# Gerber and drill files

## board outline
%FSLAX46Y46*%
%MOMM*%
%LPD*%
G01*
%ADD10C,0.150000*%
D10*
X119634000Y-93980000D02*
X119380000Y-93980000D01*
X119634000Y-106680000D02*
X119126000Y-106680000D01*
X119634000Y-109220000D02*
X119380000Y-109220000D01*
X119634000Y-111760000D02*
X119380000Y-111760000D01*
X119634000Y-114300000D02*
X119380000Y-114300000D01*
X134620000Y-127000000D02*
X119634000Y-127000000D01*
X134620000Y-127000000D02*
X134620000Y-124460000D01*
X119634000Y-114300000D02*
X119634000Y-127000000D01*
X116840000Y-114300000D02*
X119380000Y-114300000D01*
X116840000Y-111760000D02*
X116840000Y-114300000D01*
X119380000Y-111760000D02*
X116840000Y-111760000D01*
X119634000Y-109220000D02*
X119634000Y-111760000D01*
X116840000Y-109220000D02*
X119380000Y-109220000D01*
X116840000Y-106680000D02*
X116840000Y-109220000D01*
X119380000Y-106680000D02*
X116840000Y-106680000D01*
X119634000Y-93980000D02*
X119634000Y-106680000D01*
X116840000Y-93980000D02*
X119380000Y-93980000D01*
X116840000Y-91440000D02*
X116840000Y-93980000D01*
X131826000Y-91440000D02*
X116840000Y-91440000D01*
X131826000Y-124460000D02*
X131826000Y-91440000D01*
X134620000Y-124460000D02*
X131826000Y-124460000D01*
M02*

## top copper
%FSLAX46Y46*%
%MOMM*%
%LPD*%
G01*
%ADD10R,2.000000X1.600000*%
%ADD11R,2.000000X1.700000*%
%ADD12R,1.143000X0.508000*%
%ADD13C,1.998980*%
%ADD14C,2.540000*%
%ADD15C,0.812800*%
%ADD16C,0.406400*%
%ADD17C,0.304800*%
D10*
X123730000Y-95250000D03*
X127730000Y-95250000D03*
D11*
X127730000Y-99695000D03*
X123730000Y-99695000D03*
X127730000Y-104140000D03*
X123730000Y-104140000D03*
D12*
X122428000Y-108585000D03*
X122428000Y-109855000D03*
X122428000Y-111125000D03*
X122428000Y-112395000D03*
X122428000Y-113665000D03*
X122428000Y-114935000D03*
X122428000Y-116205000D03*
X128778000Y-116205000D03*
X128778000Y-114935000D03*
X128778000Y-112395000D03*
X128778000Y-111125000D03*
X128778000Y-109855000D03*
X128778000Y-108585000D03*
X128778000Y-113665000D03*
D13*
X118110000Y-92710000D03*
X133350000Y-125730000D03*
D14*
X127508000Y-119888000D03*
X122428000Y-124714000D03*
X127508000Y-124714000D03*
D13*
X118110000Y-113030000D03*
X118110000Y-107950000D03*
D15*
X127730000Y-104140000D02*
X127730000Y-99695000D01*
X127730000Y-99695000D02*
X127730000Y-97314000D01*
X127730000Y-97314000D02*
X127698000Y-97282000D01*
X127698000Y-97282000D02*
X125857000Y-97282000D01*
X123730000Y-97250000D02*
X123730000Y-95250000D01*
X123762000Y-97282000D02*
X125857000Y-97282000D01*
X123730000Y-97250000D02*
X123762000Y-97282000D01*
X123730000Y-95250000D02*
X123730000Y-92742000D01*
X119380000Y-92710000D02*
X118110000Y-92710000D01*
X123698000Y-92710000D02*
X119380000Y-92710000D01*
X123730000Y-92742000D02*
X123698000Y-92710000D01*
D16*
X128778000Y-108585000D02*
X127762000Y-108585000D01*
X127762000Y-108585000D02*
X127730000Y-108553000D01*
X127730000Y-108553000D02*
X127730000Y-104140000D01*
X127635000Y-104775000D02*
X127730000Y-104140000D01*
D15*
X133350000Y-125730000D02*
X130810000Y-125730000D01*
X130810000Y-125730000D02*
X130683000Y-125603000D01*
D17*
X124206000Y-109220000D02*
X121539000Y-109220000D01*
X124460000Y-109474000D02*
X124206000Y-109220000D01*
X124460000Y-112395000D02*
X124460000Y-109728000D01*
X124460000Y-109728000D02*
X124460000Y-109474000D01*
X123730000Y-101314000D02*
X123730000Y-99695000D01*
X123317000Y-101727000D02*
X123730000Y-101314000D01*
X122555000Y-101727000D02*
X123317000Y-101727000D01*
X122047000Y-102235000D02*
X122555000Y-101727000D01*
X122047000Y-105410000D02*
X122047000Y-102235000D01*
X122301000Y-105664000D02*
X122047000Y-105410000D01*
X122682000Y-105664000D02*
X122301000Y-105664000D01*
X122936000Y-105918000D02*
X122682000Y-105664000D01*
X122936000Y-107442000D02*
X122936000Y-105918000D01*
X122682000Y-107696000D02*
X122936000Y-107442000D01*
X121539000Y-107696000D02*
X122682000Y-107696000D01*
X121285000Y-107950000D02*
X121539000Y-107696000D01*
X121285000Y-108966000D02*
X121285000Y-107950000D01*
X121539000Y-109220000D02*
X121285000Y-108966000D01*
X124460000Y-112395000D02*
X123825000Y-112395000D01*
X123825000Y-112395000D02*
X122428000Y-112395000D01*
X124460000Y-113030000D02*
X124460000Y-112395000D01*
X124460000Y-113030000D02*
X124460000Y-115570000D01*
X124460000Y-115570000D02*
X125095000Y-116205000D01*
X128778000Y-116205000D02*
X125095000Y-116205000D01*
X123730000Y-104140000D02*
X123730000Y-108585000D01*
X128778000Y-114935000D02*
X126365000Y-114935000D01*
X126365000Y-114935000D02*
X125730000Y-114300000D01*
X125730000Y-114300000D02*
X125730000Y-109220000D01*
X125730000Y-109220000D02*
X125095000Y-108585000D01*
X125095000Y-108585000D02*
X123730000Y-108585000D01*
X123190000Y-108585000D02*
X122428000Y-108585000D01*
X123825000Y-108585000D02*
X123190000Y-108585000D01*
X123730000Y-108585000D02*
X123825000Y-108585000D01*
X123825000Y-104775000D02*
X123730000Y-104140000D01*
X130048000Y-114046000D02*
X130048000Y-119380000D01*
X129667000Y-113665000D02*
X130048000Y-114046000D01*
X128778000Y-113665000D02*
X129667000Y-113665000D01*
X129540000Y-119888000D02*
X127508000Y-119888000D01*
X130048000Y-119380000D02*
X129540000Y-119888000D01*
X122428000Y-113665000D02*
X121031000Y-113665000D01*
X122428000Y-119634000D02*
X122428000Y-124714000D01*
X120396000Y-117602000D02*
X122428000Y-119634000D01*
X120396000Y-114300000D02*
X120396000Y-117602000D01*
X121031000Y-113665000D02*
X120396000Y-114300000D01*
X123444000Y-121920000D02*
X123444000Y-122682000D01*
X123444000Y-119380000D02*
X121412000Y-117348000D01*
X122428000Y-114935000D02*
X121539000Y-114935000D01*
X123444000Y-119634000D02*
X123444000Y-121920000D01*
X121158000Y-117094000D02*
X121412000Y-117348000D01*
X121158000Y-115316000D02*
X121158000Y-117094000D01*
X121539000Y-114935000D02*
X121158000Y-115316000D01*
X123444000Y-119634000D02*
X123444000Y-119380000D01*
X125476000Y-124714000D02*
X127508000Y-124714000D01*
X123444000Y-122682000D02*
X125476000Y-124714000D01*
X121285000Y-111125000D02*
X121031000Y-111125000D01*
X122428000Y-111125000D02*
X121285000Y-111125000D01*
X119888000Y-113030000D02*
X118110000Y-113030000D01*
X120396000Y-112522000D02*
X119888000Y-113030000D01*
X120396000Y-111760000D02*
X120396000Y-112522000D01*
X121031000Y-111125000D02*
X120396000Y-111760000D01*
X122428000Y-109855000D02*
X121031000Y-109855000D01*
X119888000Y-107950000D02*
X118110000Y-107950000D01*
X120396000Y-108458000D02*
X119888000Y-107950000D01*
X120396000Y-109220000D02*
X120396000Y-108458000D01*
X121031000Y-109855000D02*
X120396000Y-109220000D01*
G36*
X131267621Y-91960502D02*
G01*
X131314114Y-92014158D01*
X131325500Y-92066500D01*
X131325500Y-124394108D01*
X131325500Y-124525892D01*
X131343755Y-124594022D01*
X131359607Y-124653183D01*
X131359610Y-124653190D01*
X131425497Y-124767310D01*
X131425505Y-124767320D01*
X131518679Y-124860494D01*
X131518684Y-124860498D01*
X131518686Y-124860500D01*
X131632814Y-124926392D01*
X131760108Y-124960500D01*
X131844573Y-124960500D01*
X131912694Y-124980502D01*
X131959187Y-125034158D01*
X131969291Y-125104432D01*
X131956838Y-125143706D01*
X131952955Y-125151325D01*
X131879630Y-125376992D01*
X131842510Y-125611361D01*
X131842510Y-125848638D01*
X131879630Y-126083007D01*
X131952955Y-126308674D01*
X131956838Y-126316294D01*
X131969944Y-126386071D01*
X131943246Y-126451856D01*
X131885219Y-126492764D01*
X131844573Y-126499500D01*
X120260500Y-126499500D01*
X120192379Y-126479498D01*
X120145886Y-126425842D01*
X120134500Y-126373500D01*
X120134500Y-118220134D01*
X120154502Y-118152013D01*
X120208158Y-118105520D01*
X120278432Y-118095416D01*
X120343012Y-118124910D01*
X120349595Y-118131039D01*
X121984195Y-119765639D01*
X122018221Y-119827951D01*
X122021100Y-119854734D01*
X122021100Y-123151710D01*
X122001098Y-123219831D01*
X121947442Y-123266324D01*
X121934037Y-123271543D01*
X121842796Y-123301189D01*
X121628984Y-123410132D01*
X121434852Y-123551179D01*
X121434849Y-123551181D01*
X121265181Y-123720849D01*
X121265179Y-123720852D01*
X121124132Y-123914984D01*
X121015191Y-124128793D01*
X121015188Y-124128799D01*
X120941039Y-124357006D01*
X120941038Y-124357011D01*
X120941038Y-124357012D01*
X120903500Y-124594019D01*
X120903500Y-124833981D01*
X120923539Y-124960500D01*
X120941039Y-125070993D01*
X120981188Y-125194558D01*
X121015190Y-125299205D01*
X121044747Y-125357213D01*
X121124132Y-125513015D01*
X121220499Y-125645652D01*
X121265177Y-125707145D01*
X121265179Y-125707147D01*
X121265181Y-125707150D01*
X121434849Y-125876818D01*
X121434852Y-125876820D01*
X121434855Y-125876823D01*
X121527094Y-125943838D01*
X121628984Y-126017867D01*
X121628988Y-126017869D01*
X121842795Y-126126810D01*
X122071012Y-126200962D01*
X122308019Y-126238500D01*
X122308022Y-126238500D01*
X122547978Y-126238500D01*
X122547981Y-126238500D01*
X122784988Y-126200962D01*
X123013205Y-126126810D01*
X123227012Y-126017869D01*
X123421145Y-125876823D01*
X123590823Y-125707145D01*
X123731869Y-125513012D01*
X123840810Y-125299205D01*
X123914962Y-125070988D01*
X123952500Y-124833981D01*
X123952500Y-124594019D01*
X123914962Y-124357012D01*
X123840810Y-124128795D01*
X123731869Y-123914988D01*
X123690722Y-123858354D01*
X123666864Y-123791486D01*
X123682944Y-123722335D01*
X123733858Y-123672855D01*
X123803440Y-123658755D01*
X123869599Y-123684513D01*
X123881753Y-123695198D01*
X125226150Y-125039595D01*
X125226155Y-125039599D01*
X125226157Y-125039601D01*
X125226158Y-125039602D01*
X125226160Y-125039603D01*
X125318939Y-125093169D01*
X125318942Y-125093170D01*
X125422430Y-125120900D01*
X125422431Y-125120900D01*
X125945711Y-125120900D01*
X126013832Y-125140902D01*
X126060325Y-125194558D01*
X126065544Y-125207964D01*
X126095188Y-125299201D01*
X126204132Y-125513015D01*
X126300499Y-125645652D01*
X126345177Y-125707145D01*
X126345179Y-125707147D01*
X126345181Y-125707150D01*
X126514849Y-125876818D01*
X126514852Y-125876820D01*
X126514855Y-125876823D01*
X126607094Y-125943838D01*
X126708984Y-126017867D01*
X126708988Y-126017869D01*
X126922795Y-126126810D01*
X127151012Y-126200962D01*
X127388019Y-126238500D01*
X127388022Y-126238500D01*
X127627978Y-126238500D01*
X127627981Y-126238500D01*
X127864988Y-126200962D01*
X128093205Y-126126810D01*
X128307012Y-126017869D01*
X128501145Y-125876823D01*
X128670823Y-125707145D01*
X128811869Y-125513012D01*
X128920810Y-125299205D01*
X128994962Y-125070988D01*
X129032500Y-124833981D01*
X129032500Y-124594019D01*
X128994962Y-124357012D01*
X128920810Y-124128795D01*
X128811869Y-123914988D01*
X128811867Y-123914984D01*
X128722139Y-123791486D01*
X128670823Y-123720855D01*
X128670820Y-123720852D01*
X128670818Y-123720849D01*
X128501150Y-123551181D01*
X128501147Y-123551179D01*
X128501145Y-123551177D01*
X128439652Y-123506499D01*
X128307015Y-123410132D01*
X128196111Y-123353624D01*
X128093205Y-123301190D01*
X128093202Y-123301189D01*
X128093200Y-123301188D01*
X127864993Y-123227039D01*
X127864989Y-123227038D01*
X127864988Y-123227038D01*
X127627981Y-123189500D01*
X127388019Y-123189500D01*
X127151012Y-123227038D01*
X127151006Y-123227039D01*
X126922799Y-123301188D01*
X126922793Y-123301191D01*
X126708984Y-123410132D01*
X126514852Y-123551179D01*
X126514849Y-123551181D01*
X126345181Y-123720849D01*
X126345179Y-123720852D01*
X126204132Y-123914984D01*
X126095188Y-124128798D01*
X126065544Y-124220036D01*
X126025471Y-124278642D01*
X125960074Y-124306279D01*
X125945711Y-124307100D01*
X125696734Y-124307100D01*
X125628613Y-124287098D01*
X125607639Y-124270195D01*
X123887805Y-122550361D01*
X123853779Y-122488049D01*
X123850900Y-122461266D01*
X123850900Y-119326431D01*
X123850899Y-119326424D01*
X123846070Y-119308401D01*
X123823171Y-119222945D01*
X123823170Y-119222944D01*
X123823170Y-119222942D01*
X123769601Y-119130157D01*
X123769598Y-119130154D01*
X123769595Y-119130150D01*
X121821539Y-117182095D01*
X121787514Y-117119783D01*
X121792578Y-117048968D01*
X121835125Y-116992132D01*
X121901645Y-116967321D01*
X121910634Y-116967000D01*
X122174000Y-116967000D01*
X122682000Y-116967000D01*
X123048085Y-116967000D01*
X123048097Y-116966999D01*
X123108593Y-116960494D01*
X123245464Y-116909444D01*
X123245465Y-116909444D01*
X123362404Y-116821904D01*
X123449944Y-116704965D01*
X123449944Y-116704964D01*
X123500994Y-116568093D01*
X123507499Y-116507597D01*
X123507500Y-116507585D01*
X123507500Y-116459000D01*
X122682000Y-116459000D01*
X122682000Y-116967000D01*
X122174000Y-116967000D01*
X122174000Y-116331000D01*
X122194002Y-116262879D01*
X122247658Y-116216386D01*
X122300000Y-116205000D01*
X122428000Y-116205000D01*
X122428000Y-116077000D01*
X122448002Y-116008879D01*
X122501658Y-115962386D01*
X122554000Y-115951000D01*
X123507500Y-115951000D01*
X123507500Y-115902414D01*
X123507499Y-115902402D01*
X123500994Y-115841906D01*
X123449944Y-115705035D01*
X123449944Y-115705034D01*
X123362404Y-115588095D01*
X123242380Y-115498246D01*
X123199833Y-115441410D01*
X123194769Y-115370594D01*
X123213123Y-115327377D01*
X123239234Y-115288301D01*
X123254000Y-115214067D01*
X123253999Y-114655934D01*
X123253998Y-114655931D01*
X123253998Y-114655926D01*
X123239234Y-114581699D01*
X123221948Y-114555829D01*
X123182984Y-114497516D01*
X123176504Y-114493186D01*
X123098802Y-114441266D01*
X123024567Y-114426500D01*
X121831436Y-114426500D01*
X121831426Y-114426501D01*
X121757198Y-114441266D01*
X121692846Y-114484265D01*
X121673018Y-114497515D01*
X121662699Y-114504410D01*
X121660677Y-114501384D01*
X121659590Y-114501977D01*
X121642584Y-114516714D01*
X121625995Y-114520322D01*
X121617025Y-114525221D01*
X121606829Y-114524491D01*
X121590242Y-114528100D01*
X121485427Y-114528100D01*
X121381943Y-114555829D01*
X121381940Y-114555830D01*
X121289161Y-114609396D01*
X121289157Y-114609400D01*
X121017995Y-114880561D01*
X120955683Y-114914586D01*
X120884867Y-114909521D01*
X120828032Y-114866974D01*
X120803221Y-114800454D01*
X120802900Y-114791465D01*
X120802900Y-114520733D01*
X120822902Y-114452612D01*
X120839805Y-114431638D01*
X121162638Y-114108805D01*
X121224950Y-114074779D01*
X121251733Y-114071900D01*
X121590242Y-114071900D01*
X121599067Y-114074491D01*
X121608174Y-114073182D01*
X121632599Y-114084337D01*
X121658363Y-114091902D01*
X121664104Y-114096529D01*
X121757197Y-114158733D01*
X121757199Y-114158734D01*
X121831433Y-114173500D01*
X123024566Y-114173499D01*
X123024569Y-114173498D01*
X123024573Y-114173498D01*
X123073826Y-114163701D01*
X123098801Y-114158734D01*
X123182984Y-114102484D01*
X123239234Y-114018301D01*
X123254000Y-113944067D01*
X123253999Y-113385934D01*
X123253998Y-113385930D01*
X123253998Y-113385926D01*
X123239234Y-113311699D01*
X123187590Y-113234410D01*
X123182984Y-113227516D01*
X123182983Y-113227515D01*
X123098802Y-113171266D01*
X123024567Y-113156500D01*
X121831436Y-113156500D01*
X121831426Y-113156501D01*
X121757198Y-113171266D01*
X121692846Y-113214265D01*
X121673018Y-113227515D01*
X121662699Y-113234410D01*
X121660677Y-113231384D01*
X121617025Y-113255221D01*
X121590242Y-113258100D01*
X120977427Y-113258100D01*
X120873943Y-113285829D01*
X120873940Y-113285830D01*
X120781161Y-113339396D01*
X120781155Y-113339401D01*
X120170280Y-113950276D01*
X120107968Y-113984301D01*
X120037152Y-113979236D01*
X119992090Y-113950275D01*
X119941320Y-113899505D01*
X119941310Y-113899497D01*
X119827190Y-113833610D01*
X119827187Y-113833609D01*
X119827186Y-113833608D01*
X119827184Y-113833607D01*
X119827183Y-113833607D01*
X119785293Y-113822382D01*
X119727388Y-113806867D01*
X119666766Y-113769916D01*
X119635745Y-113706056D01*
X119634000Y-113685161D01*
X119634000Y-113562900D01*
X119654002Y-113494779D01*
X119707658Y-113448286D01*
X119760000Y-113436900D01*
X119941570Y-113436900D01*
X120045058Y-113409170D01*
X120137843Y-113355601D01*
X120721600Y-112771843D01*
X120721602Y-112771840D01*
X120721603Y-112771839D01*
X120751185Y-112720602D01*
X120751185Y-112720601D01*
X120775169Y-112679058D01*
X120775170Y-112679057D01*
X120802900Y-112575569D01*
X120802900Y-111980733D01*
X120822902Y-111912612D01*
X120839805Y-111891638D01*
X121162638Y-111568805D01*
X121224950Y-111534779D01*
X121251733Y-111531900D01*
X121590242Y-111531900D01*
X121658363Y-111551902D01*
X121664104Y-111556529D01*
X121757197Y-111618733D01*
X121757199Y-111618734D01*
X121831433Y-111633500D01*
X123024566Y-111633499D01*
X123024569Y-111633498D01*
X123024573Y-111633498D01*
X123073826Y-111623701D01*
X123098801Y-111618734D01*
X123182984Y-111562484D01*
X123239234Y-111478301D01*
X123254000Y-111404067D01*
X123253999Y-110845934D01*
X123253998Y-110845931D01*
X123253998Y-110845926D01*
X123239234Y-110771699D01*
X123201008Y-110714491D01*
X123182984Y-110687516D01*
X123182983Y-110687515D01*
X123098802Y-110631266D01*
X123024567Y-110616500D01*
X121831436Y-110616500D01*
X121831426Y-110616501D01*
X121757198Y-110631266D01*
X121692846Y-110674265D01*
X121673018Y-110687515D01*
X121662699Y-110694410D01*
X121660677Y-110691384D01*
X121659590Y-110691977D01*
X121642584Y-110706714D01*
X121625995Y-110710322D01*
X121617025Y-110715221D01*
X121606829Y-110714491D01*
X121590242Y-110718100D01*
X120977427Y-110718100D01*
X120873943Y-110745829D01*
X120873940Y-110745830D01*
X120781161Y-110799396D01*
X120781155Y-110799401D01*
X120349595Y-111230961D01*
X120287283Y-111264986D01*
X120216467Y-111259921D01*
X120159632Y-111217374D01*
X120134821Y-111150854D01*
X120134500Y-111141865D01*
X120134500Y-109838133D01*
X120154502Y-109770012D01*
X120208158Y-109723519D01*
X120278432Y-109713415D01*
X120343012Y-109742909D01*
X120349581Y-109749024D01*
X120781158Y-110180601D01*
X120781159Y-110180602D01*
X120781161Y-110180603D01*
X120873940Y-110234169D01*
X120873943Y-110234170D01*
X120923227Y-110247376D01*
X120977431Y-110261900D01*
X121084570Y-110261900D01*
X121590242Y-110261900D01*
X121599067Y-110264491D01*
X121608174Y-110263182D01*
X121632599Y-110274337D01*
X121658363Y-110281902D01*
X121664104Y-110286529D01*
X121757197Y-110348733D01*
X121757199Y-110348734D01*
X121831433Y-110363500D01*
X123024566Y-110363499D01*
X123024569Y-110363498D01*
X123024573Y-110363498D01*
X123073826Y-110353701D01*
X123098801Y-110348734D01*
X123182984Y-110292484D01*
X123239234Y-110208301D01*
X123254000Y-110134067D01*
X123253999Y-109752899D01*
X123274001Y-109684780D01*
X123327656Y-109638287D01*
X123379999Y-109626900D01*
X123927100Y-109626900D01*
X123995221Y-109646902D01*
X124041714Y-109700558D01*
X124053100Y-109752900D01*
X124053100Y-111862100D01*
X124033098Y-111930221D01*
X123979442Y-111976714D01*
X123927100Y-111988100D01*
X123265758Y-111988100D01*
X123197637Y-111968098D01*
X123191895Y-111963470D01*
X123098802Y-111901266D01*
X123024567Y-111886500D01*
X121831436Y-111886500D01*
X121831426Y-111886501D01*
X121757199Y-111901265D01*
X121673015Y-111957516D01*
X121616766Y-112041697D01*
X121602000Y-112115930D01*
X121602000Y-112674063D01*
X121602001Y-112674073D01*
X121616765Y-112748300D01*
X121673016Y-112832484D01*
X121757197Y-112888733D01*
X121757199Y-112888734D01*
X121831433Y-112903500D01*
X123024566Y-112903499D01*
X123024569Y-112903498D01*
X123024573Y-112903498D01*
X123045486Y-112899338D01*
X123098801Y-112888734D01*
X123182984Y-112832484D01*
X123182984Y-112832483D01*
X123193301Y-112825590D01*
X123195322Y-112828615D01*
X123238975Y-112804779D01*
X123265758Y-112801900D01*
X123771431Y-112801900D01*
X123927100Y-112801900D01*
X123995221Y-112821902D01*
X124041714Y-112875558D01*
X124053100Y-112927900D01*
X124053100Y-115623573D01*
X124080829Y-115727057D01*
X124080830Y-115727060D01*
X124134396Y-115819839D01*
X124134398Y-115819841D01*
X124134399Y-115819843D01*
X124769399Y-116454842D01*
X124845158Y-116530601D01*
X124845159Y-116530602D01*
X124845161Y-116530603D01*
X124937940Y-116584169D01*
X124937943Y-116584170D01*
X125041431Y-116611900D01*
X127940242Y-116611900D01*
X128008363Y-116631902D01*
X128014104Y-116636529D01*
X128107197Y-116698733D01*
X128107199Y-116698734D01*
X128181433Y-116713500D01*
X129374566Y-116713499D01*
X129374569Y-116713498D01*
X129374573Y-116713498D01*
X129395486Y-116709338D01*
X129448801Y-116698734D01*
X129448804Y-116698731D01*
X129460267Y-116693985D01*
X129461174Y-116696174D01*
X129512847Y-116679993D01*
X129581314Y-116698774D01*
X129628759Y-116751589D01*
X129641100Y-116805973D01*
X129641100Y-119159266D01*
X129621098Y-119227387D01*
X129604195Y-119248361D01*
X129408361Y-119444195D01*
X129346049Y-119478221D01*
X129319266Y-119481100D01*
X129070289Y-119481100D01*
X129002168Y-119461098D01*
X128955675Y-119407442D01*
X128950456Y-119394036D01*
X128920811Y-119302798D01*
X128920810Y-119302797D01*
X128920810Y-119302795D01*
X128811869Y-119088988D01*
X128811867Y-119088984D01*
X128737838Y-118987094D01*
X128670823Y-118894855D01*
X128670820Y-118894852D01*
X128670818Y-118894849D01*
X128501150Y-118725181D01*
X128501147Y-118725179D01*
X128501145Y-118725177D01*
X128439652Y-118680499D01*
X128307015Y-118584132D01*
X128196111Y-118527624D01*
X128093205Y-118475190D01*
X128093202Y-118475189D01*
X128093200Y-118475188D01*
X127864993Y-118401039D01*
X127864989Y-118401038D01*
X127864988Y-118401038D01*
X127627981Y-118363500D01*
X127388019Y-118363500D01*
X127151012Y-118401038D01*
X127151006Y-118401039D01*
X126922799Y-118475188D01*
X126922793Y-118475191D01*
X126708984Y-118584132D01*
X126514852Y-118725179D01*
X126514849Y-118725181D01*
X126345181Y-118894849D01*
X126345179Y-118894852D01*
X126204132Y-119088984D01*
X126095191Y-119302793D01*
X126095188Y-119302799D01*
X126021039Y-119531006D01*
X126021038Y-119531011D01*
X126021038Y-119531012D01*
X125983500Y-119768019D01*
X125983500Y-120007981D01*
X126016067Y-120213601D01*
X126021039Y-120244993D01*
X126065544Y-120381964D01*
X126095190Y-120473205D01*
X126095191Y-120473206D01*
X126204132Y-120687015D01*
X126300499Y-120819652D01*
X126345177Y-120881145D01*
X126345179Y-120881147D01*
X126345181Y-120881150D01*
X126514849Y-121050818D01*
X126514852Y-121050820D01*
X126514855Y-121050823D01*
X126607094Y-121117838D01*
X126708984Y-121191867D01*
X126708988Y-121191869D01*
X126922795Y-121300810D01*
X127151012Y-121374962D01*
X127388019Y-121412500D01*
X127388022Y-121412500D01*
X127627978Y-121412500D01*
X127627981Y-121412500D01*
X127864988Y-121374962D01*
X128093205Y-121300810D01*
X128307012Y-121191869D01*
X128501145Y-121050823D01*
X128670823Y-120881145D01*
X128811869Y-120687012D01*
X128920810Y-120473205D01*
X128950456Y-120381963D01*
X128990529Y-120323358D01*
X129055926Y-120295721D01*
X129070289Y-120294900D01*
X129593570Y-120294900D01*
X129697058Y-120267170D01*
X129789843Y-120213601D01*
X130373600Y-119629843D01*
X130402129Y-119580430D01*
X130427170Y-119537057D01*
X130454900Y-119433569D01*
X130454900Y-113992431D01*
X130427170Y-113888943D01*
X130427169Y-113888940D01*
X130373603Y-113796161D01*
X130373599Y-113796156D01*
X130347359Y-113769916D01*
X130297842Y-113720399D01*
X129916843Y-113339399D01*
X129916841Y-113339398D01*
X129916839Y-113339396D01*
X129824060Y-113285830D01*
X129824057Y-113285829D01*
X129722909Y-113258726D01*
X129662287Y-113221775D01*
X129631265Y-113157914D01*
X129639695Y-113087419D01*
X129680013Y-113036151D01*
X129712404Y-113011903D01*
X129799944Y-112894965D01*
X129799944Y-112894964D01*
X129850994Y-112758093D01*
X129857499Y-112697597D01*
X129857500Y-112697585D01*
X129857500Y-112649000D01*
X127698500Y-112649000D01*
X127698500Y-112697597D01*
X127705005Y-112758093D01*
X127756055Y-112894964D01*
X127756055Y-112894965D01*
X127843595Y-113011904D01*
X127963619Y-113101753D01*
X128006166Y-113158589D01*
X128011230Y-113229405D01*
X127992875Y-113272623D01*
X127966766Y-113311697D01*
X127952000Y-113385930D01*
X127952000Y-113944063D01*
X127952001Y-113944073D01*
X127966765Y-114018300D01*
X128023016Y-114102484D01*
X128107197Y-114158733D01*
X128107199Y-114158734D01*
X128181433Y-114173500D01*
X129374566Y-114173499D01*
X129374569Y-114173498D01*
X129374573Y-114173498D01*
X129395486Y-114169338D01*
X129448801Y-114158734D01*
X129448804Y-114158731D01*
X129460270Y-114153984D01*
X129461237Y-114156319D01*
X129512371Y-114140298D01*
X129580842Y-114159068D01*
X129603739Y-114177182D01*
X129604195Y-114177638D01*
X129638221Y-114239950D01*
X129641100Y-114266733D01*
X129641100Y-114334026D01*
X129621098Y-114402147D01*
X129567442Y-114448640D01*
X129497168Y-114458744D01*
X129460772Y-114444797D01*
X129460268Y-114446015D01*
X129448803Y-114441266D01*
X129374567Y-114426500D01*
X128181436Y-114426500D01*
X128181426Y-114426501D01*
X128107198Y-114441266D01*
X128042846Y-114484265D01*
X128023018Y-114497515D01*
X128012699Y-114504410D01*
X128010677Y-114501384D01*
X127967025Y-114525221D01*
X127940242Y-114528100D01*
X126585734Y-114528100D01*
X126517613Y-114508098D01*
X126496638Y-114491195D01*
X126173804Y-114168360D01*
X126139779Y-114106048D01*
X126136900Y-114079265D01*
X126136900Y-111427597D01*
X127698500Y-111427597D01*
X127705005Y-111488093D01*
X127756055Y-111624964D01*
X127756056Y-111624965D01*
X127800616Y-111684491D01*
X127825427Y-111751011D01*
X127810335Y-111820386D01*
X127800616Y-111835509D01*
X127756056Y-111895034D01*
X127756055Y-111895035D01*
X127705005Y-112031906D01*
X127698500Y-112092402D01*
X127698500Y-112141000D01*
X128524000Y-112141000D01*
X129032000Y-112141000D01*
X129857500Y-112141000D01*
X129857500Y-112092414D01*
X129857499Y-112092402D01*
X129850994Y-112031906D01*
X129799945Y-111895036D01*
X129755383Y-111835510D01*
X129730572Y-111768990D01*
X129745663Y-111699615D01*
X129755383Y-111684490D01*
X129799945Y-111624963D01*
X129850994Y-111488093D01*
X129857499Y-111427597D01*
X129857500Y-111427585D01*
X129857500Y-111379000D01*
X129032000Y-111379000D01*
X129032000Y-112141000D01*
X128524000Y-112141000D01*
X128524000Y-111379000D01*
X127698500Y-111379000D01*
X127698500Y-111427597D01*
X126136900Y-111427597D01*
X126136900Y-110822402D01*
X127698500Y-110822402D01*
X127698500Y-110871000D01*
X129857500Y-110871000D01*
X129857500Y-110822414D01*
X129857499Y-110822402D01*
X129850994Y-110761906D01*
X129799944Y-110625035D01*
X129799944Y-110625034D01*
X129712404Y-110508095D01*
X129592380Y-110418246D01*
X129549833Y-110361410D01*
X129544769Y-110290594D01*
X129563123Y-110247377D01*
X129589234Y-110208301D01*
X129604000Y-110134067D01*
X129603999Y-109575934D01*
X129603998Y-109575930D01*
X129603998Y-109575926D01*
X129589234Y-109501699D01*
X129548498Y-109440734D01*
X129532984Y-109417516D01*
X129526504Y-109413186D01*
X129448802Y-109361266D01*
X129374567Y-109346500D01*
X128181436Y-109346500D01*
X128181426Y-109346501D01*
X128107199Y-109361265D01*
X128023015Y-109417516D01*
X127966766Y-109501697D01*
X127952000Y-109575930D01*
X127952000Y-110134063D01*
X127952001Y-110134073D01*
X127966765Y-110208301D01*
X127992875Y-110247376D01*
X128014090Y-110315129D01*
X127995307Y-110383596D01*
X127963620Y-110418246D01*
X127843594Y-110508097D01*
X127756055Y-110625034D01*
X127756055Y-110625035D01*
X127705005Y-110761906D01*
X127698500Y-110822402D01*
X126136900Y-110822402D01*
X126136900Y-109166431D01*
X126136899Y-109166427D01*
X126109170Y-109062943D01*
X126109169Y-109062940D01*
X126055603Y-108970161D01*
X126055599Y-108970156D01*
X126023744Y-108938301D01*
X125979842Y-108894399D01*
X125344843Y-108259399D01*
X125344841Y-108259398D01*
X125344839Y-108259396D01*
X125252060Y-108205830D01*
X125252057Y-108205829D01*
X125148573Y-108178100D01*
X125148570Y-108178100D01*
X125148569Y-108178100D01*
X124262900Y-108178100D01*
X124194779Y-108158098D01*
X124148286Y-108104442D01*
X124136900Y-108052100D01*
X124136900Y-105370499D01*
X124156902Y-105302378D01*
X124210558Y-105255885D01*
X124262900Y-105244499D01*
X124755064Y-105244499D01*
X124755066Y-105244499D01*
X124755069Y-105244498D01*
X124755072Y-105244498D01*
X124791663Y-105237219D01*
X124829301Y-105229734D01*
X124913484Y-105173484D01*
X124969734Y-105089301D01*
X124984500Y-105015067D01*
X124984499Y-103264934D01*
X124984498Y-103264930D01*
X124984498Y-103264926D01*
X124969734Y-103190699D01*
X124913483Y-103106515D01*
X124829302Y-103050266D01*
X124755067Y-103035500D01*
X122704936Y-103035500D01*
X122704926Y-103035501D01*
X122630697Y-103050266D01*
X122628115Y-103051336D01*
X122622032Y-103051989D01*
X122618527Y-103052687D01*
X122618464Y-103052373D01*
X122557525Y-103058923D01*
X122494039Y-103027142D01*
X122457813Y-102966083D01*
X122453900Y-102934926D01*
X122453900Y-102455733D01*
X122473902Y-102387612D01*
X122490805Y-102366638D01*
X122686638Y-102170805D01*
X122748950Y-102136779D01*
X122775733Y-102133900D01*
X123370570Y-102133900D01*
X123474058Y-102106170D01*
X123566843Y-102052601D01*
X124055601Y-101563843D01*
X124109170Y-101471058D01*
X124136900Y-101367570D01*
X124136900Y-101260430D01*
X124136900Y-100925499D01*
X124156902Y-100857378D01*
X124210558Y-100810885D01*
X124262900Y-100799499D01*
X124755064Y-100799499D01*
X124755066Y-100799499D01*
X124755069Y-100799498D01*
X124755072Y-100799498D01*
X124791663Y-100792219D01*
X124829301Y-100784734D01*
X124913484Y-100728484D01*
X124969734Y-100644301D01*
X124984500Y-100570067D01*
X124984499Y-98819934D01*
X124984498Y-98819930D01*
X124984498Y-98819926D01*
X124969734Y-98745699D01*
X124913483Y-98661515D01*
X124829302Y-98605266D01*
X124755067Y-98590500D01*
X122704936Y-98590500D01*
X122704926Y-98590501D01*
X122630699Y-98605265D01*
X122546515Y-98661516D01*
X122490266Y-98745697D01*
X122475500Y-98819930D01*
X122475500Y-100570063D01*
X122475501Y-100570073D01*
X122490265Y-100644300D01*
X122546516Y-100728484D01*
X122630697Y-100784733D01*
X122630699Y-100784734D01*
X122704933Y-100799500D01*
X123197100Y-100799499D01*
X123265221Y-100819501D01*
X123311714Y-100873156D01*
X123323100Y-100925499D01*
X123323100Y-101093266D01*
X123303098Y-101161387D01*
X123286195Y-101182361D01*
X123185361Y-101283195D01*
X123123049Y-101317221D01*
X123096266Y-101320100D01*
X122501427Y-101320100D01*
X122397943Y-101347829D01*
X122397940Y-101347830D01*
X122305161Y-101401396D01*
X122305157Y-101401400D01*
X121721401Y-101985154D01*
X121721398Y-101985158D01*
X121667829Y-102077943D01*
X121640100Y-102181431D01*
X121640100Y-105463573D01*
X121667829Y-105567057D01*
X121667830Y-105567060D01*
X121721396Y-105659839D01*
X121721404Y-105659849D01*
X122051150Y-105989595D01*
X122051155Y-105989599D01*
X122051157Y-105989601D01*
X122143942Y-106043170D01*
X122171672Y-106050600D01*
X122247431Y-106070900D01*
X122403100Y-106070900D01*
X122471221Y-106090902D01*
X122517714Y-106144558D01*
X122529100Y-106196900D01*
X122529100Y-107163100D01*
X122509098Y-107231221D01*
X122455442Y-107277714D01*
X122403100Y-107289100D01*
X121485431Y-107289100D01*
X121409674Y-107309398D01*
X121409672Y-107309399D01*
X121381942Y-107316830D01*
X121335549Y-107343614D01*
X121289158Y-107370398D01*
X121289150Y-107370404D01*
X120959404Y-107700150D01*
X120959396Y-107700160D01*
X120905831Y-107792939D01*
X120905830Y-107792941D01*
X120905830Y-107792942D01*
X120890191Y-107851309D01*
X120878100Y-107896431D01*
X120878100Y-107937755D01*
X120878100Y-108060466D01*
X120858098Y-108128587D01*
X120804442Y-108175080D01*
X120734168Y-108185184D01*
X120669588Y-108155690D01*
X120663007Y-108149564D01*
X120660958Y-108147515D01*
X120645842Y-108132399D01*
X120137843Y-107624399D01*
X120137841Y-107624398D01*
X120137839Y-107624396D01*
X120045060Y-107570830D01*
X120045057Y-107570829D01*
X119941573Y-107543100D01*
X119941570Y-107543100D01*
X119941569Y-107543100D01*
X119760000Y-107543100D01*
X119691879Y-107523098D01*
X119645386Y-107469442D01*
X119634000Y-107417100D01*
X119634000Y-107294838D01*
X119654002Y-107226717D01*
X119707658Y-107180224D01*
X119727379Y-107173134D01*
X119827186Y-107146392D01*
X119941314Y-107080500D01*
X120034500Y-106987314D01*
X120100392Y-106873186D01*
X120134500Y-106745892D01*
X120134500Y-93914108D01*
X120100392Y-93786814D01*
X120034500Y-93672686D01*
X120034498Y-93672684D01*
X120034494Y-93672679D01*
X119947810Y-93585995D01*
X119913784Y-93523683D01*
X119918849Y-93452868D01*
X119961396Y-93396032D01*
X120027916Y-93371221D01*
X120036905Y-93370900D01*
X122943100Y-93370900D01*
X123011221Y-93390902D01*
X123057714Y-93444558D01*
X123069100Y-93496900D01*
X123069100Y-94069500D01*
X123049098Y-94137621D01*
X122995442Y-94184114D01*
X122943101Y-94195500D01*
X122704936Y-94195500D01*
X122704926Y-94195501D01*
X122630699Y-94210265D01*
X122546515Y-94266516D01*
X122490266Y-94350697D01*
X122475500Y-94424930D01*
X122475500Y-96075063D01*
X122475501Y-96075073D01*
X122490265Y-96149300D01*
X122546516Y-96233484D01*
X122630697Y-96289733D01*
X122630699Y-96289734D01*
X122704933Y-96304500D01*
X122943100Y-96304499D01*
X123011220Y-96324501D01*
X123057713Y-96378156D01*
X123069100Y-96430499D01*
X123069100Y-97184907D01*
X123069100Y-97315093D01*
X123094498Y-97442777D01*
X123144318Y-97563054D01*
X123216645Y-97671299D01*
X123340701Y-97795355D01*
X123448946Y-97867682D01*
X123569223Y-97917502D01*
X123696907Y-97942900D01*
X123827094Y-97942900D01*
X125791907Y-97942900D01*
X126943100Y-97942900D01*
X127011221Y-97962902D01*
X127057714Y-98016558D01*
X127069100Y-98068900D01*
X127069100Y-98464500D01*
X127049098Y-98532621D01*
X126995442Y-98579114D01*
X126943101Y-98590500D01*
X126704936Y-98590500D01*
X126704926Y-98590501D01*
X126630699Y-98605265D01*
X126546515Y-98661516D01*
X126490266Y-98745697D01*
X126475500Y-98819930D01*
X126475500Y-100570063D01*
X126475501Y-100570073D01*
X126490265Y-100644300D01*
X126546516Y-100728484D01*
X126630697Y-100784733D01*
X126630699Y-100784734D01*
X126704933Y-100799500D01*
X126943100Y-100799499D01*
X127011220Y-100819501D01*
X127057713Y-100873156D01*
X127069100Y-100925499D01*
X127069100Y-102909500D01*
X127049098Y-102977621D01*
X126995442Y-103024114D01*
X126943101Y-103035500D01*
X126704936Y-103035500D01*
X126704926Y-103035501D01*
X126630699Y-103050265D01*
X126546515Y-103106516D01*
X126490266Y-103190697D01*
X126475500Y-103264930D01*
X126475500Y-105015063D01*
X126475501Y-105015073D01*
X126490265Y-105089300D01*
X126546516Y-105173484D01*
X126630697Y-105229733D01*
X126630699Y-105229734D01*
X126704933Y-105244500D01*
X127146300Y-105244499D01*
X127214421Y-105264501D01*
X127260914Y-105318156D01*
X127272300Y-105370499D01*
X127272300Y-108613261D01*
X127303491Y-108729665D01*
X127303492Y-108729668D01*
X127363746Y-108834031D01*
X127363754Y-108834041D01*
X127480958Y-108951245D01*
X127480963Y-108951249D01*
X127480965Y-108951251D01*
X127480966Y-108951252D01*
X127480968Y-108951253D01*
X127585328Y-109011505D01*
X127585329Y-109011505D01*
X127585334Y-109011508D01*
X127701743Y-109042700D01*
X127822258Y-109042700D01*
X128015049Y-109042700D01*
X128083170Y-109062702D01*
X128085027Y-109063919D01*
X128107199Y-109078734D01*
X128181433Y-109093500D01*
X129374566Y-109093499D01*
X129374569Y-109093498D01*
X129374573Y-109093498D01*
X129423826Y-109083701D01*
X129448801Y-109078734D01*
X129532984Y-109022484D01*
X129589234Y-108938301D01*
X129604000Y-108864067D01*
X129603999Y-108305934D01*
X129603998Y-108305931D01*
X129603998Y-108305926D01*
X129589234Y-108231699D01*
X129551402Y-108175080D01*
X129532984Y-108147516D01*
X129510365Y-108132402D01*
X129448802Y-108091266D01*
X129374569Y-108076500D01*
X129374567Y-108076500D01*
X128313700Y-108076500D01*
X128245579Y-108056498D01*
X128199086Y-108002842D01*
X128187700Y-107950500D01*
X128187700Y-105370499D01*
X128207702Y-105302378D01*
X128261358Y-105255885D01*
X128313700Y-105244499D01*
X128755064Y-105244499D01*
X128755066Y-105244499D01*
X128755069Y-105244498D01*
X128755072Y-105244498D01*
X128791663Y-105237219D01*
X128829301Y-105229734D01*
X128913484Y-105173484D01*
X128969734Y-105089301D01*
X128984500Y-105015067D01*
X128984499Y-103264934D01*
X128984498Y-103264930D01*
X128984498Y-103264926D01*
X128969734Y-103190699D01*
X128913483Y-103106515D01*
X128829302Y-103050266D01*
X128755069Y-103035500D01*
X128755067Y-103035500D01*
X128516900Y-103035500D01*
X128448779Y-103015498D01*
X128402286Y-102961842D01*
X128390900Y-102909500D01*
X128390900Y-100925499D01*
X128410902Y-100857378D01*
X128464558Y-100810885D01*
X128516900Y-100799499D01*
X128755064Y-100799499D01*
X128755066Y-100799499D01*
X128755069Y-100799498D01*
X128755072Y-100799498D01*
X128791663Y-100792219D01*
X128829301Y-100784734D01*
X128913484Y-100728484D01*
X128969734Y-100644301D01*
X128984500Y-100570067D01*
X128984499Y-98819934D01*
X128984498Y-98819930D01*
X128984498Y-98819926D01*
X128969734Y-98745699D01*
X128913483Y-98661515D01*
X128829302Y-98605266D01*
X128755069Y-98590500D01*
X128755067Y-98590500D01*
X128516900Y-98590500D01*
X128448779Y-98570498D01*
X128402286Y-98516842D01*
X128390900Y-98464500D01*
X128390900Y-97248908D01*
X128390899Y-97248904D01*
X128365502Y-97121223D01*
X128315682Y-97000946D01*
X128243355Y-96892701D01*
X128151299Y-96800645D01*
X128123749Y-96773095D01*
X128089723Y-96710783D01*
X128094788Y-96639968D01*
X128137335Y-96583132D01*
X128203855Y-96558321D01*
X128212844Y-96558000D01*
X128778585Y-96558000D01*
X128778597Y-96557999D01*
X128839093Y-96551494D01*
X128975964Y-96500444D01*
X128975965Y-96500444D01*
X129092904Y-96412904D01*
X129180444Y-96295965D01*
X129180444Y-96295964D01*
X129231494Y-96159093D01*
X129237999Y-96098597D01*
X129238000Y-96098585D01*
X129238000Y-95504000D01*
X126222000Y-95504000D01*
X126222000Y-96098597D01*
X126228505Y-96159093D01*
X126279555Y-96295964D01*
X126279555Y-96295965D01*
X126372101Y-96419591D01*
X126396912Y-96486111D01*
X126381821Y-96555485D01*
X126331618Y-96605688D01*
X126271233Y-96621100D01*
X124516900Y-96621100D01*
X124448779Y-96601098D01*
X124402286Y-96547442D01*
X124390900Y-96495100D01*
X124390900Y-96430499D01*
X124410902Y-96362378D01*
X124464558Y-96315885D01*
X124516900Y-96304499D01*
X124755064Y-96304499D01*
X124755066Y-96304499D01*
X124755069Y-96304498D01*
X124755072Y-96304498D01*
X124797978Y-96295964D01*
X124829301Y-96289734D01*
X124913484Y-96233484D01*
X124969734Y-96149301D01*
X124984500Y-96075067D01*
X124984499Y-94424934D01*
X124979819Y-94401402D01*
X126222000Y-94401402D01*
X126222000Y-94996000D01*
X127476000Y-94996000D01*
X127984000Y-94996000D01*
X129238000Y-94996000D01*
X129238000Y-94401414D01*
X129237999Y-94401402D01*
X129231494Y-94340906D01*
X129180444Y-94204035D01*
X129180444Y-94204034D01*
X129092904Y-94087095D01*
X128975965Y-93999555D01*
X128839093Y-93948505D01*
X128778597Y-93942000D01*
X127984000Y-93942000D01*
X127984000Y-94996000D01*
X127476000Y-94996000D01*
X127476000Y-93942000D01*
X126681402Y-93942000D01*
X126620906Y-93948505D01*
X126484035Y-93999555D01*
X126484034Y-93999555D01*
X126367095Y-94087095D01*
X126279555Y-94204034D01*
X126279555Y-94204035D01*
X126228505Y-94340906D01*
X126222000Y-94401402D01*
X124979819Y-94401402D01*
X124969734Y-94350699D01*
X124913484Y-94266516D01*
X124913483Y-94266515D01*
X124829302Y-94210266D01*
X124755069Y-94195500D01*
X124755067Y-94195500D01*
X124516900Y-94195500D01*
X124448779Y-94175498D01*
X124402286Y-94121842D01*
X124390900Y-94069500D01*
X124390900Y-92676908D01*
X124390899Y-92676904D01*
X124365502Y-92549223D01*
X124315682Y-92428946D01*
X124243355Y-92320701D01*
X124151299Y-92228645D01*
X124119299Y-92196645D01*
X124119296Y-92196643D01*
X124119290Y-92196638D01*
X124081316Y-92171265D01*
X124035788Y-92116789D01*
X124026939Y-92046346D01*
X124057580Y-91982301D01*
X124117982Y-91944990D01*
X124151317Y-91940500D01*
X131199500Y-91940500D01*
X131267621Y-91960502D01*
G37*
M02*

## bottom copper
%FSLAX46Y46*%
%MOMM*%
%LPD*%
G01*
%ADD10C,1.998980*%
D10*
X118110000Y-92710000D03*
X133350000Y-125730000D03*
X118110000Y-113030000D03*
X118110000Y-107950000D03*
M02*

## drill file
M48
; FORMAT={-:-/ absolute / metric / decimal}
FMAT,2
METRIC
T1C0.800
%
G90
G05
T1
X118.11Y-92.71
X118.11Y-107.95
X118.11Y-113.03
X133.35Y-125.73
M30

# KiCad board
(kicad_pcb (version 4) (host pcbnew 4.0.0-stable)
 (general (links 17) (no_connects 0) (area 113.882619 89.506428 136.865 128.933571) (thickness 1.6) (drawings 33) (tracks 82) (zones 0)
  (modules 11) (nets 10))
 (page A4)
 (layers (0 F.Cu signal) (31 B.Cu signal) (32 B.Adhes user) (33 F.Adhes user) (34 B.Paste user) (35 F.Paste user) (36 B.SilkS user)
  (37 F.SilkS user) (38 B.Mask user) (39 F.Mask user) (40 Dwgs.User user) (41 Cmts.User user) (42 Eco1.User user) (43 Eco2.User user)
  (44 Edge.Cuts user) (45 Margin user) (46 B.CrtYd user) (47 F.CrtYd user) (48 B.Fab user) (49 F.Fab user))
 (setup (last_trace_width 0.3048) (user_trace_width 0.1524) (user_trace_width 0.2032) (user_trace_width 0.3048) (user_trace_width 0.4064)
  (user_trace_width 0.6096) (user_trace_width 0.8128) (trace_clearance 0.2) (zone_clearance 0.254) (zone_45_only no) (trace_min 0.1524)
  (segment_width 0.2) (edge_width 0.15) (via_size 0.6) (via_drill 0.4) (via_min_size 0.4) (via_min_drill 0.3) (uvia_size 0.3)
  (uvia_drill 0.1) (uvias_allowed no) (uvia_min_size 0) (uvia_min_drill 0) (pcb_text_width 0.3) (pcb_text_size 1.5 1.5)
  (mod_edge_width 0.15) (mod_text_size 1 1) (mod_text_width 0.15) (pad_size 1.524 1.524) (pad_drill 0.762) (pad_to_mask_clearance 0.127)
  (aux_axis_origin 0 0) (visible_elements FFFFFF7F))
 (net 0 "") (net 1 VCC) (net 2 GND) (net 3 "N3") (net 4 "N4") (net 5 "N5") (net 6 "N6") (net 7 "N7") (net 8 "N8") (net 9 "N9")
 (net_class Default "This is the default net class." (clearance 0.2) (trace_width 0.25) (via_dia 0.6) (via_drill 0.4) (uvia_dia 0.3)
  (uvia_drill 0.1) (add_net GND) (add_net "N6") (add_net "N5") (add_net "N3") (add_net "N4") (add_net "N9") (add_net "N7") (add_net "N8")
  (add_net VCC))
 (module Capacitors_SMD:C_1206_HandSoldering (layer F.Cu) (at 125.73 95.25)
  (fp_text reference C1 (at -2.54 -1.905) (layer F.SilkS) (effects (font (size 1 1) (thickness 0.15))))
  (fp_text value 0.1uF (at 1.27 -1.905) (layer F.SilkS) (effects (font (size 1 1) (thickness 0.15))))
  (pad 1 smd rect (at -2 0) (size 2 1.6) (layers F.Cu F.Paste F.Mask) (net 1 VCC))
  (pad 2 smd rect (at 2 0) (size 2 1.6) (layers F.Cu F.Paste F.Mask) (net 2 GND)))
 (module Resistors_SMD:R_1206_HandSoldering (layer F.Cu) (at 125.73 99.695 180)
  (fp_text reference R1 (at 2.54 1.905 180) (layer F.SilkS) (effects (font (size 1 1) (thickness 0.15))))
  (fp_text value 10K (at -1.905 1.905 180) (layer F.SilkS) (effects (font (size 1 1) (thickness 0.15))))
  (pad 1 smd rect (at -2 0 180) (size 2 1.7) (layers F.Cu F.Paste F.Mask) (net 1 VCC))
  (pad 2 smd rect (at 2 0 180) (size 2 1.7) (layers F.Cu F.Paste F.Mask) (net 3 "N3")))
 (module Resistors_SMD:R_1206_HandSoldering (layer F.Cu) (at 125.73 104.14 180)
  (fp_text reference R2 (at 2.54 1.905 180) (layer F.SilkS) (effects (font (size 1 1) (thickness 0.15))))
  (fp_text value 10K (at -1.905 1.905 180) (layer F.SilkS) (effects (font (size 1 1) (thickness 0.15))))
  (pad 1 smd rect (at -2 0 180) (size 2 1.7) (layers F.Cu F.Paste F.Mask) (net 1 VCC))
  (pad 2 smd rect (at 2 0 180) (size 2 1.7) (layers F.Cu F.Paste F.Mask) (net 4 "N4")))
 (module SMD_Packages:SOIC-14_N (layer F.Cu) (at 125.73 112.395 270)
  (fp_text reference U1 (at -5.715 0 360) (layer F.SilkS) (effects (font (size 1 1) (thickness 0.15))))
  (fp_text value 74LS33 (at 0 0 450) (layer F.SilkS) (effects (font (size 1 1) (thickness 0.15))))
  (pad 1 smd rect (at -3.81 3.302 270) (size 0.508 1.143) (layers F.Cu F.Paste F.Mask) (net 4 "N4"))
  (pad 2 smd rect (at -2.54 3.302 270) (size 0.508 1.143) (layers F.Cu F.Paste F.Mask) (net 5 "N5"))
  (pad 3 smd rect (at -1.27 3.302 270) (size 0.508 1.143) (layers F.Cu F.Paste F.Mask) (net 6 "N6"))
  (pad 4 smd rect (at 0 3.302 270) (size 0.508 1.143) (layers F.Cu F.Paste F.Mask) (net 3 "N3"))
  (pad 5 smd rect (at 1.27 3.302 270) (size 0.508 1.143) (layers F.Cu F.Paste F.Mask) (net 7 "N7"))
  (pad 6 smd rect (at 2.54 3.302 270) (size 0.508 1.143) (layers F.Cu F.Paste F.Mask) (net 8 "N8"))
  (pad 7 smd rect (at 3.81 3.302 270) (size 0.508 1.143) (layers F.Cu F.Paste F.Mask) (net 2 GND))
  (pad 8 smd rect (at 3.81 -3.048 270) (size 0.508 1.143) (layers F.Cu F.Paste F.Mask) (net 3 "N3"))
  (pad 9 smd rect (at 2.54 -3.048 270) (size 0.508 1.143) (layers F.Cu F.Paste F.Mask) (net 4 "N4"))
  (pad 11 smd rect (at 0 -3.048 270) (size 0.508 1.143) (layers F.Cu F.Paste F.Mask) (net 2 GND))
  (pad 12 smd rect (at -1.27 -3.048 270) (size 0.508 1.143) (layers F.Cu F.Paste F.Mask) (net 2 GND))
  (pad 13 smd rect (at -2.54 -3.048 270) (size 0.508 1.143) (layers F.Cu F.Paste F.Mask))
  (pad 14 smd rect (at -3.81 -3.048 270) (size 0.508 1.143) (layers F.Cu F.Paste F.Mask) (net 1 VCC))
  (pad 10 smd rect (at 1.27 -3.048 270) (size 0.508 1.143) (layers F.Cu F.Paste F.Mask) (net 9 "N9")))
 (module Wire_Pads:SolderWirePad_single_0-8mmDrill (layer F.Cu) (at 118.11 92.71 90)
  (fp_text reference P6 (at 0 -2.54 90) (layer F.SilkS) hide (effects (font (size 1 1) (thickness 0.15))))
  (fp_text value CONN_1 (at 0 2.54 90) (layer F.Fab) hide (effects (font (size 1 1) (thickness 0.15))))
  (pad 1 thru_hole circle (at 0 0 90) (size 1.99898 1.99898) (drill 0.8001) (layers *.Cu *.Mask F.SilkS) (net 1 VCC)))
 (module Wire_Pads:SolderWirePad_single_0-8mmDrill (layer F.Cu) (at 133.35 125.73 270)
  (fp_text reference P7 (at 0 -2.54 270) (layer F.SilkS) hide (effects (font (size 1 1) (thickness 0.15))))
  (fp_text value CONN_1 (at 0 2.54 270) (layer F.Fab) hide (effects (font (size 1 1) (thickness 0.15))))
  (pad 1 thru_hole circle (at 0 0 270) (size 1.99898 1.99898) (drill 0.8001) (layers *.Cu *.Mask F.SilkS) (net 2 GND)))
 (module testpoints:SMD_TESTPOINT (layer F.Cu) (at 127.508 119.888)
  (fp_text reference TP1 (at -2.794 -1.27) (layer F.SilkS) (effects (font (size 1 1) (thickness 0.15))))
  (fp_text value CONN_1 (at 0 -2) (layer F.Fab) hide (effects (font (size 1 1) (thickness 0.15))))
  (pad 1 smd circle (at 0 0) (size 2.54 2.54) (layers F.Cu F.Paste F.Mask) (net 9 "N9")))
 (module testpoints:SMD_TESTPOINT (layer F.Cu) (at 122.428 124.714)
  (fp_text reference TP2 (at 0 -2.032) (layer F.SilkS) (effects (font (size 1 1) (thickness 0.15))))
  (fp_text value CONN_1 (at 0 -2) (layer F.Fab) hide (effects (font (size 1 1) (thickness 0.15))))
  (pad 1 smd circle (at 0 0) (size 2.54 2.54) (layers F.Cu F.Paste F.Mask) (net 7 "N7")))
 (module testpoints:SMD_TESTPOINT (layer F.Cu) (at 127.508 124.714)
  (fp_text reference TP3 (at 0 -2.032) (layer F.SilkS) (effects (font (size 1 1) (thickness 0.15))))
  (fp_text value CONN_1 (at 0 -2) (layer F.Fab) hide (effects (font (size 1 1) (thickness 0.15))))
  (pad 1 smd circle (at 0 0) (size 2.54 2.54) (layers F.Cu F.Paste F.Mask) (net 8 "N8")))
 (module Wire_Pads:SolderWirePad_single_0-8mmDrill (layer F.Cu) (at 118.11 113.03)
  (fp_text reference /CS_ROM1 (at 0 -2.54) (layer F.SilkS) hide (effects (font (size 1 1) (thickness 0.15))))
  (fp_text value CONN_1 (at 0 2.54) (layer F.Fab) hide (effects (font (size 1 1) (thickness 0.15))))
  (pad 1 thru_hole circle (at 0 0) (size 1.99898 1.99898) (drill 0.8001) (layers *.Cu *.Mask F.SilkS) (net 6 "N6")))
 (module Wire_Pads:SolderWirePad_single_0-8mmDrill (layer F.Cu) (at 118.11 107.95)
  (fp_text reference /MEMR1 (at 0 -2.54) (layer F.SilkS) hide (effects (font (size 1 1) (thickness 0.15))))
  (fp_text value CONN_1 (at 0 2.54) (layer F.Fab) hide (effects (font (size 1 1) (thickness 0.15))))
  (pad 1 thru_hole circle (at 0 0) (size 1.99898 1.99898) (drill 0.8001) (layers *.Cu *.Mask F.SilkS) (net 5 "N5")))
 (gr_line (start 119.634 93.98) (end 119.38 93.98) (angle 90) (layer Edge.Cuts) (width 0.15))
 (gr_line (start 119.634 106.68) (end 119.126 106.68) (angle 90) (layer Edge.Cuts) (width 0.15))
 (gr_line (start 119.634 109.22) (end 119.38 109.22) (angle 90) (layer Edge.Cuts) (width 0.15))
 (gr_line (start 119.634 111.76) (end 119.38 111.76) (angle 90) (layer Edge.Cuts) (width 0.15))
 (gr_line (start 119.634 114.3) (end 119.38 114.3) (angle 90) (layer Edge.Cuts) (width 0.15))
 (gr_line (start 134.62 127) (end 119.634 127) (angle 90) (layer Edge.Cuts) (width 0.15))
 (gr_line (start 134.62 127) (end 134.62 124.46) (angle 90) (layer Edge.Cuts) (width 0.15))
 (gr_line (start 119.634 114.3) (end 119.634 127) (angle 90) (layer Edge.Cuts) (width 0.15))
 (gr_line (start 116.84 114.3) (end 119.38 114.3) (angle 90) (layer Edge.Cuts) (width 0.15))
 (gr_line (start 116.84 111.76) (end 116.84 114.3) (angle 90) (layer Edge.Cuts) (width 0.15))
 (gr_line (start 119.38 111.76) (end 116.84 111.76) (angle 90) (layer Edge.Cuts) (width 0.15))
 (gr_line (start 119.634 109.22) (end 119.634 111.76) (angle 90) (layer Edge.Cuts) (width 0.15))
 (gr_line (start 116.84 109.22) (end 119.38 109.22) (angle 90) (layer Edge.Cuts) (width 0.15))
 (gr_line (start 116.84 106.68) (end 116.84 109.22) (angle 90) (layer Edge.Cuts) (width 0.15))
 (gr_line (start 119.38 106.68) (end 116.84 106.68) (angle 90) (layer Edge.Cuts) (width 0.15))
 (gr_line (start 119.634 93.98) (end 119.634 106.68) (angle 90) (layer Edge.Cuts) (width 0.15))
 (gr_line (start 116.84 93.98) (end 119.38 93.98) (angle 90) (layer Edge.Cuts) (width 0.15))
 (gr_line (start 116.84 91.44) (end 116.84 93.98) (angle 90) (layer Edge.Cuts) (width 0.15))
 (gr_line (start 131.826 91.44) (end 116.84 91.44) (angle 90) (layer Edge.Cuts) (width 0.15))
 (gr_line (start 131.826 124.46) (end 131.826 91.44) (angle 90) (layer Edge.Cuts) (width 0.15))
 (gr_line (start 134.62 124.46) (end 131.826 124.46) (angle 90) (layer Edge.Cuts) (width 0.15))
 (segment (start 127.73 104.14) (end 127.73 99.695) (width 0.8128) (layer F.Cu) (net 1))
 (segment (start 127.73 99.695) (end 127.73 97.314) (width 0.8128) (layer F.Cu) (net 1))
 (segment (start 127.73 97.314) (end 127.698 97.282) (width 0.8128) (layer F.Cu) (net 1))
 (segment (start 127.698 97.282) (end 125.857 97.282) (width 0.8128) (layer F.Cu) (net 1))
 (segment (start 123.73 97.25) (end 123.73 95.25) (width 0.8128) (layer F.Cu) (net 1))
 (segment (start 123.762 97.282) (end 125.857 97.282) (width 0.8128) (layer F.Cu) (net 1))
 (segment (start 123.73 97.25) (end 123.762 97.282) (width 0.8128) (layer F.Cu) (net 1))
 (segment (start 123.73 95.25) (end 123.73 92.742) (width 0.8128) (layer F.Cu) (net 1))
 (segment (start 119.38 92.71) (end 118.11 92.71) (width 0.8128) (layer F.Cu) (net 1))
 (segment (start 123.698 92.71) (end 119.38 92.71) (width 0.8128) (layer F.Cu) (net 1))
 (segment (start 123.73 92.742) (end 123.698 92.71) (width 0.8128) (layer F.Cu) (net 1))
 (segment (start 128.778 108.585) (end 127.762 108.585) (width 0.4064) (layer F.Cu) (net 1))
 (segment (start 127.762 108.585) (end 127.73 108.553) (width 0.4064) (layer F.Cu) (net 1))
 (segment (start 127.73 108.553) (end 127.73 104.14) (width 0.4064) (layer F.Cu) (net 1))
 (segment (start 127.635 104.775) (end 127.73 104.14) (width 0.4064) (layer F.Cu) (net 1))
 (segment (start 133.35 125.73) (end 130.81 125.73) (width 0.8128) (layer F.Cu) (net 2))
 (segment (start 130.81 125.73) (end 130.683 125.603) (width 0.8128) (layer F.Cu) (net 2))
 (segment (start 124.206 109.22) (end 121.539 109.22) (width 0.3048) (layer F.Cu) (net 3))
 (segment (start 124.46 109.474) (end 124.206 109.22) (width 0.3048) (layer F.Cu) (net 3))
 (segment (start 124.46 112.395) (end 124.46 109.728) (width 0.3048) (layer F.Cu) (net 3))
 (segment (start 124.46 109.728) (end 124.46 109.474) (width 0.3048) (layer F.Cu) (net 3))
 (segment (start 123.73 101.314) (end 123.73 99.695) (width 0.3048) (layer F.Cu) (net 3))
 (segment (start 123.317 101.727) (end 123.73 101.314) (width 0.3048) (layer F.Cu) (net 3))
 (segment (start 122.555 101.727) (end 123.317 101.727) (width 0.3048) (layer F.Cu) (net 3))
 (segment (start 122.047 102.235) (end 122.555 101.727) (width 0.3048) (layer F.Cu) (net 3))
 (segment (start 122.047 105.41) (end 122.047 102.235) (width 0.3048) (layer F.Cu) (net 3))
 (segment (start 122.301 105.664) (end 122.047 105.41) (width 0.3048) (layer F.Cu) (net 3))
 (segment (start 122.682 105.664) (end 122.301 105.664) (width 0.3048) (layer F.Cu) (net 3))
 (segment (start 122.936 105.918) (end 122.682 105.664) (width 0.3048) (layer F.Cu) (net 3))
 (segment (start 122.936 107.442) (end 122.936 105.918) (width 0.3048) (layer F.Cu) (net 3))
 (segment (start 122.682 107.696) (end 122.936 107.442) (width 0.3048) (layer F.Cu) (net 3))
 (segment (start 121.539 107.696) (end 122.682 107.696) (width 0.3048) (layer F.Cu) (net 3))
 (segment (start 121.285 107.95) (end 121.539 107.696) (width 0.3048) (layer F.Cu) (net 3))
 (segment (start 121.285 108.966) (end 121.285 107.95) (width 0.3048) (layer F.Cu) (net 3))
 (segment (start 121.539 109.22) (end 121.285 108.966) (width 0.3048) (layer F.Cu) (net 3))
 (segment (start 124.46 112.395) (end 123.825 112.395) (width 0.3048) (layer F.Cu) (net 3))
 (segment (start 123.825 112.395) (end 122.428 112.395) (width 0.3048) (layer F.Cu) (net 3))
 (segment (start 124.46 113.03) (end 124.46 112.395) (width 0.3048) (layer F.Cu) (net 3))
 (segment (start 124.46 113.03) (end 124.46 115.57) (width 0.3048) (layer F.Cu) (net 3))
 (segment (start 124.46 115.57) (end 125.095 116.205) (width 0.3048) (layer F.Cu) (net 3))
 (segment (start 128.778 116.205) (end 125.095 116.205) (width 0.3048) (layer F.Cu) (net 3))
 (segment (start 123.73 104.14) (end 123.73 108.585) (width 0.3048) (layer F.Cu) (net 4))
 (segment (start 128.778 114.935) (end 126.365 114.935) (width 0.3048) (layer F.Cu) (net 4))
 (segment (start 126.365 114.935) (end 125.73 114.3) (width 0.3048) (layer F.Cu) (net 4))
 (segment (start 125.73 114.3) (end 125.73 109.22) (width 0.3048) (layer F.Cu) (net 4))
 (segment (start 125.73 109.22) (end 125.095 108.585) (width 0.3048) (layer F.Cu) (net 4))
 (segment (start 125.095 108.585) (end 123.73 108.585) (width 0.3048) (layer F.Cu) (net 4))
 (segment (start 123.19 108.585) (end 122.428 108.585) (width 0.3048) (layer F.Cu) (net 4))
 (segment (start 123.825 108.585) (end 123.19 108.585) (width 0.3048) (layer F.Cu) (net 4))
 (segment (start 123.73 108.585) (end 123.825 108.585) (width 0.3048) (layer F.Cu) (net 4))
 (segment (start 123.825 104.775) (end 123.73 104.14) (width 0.3048) (layer F.Cu) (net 4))
 (segment (start 130.048 114.046) (end 130.048 119.38) (width 0.3048) (layer F.Cu) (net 9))
 (segment (start 129.667 113.665) (end 130.048 114.046) (width 0.3048) (layer F.Cu) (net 9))
 (segment (start 128.778 113.665) (end 129.667 113.665) (width 0.3048) (layer F.Cu) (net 9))
 (segment (start 129.54 119.888) (end 127.508 119.888) (width 0.3048) (layer F.Cu) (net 9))
 (segment (start 130.048 119.38) (end 129.54 119.888) (width 0.3048) (layer F.Cu) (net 9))
 (segment (start 122.428 113.665) (end 121.031 113.665) (width 0.3048) (layer F.Cu) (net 7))
 (segment (start 122.428 119.634) (end 122.428 124.714) (width 0.3048) (layer F.Cu) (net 7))
 (segment (start 120.396 117.602) (end 122.428 119.634) (width 0.3048) (layer F.Cu) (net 7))
 (segment (start 120.396 114.3) (end 120.396 117.602) (width 0.3048) (layer F.Cu) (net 7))
 (segment (start 121.031 113.665) (end 120.396 114.3) (width 0.3048) (layer F.Cu) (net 7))
 (segment (start 123.444 121.92) (end 123.444 122.682) (width 0.3048) (layer F.Cu) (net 8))
 (segment (start 123.444 119.38) (end 121.412 117.348) (width 0.3048) (layer F.Cu) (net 8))
 (segment (start 122.428 114.935) (end 121.539 114.935) (width 0.3048) (layer F.Cu) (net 8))
 (segment (start 123.444 119.634) (end 123.444 121.92) (width 0.3048) (layer F.Cu) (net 8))
 (segment (start 121.158 117.094) (end 121.412 117.348) (width 0.3048) (layer F.Cu) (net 8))
 (segment (start 121.158 115.316) (end 121.158 117.094) (width 0.3048) (layer F.Cu) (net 8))
 (segment (start 121.539 114.935) (end 121.158 115.316) (width 0.3048) (layer F.Cu) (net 8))
 (segment (start 123.444 119.634) (end 123.444 119.38) (width 0.3048) (layer F.Cu) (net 8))
 (segment (start 125.476 124.714) (end 127.508 124.714) (width 0.3048) (layer F.Cu) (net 8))
 (segment (start 123.444 122.682) (end 125.476 124.714) (width 0.3048) (layer F.Cu) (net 8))
 (segment (start 121.285 111.125) (end 121.031 111.125) (width 0.3048) (layer F.Cu) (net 6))
 (segment (start 122.428 111.125) (end 121.285 111.125) (width 0.3048) (layer F.Cu) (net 6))
 (segment (start 119.888 113.03) (end 118.11 113.03) (width 0.3048) (layer F.Cu) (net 6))
 (segment (start 120.396 112.522) (end 119.888 113.03) (width 0.3048) (layer F.Cu) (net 6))
 (segment (start 120.396 111.76) (end 120.396 112.522) (width 0.3048) (layer F.Cu) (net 6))
 (segment (start 121.031 111.125) (end 120.396 111.76) (width 0.3048) (layer F.Cu) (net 6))
 (segment (start 122.428 109.855) (end 121.031 109.855) (width 0.3048) (layer F.Cu) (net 5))
 (segment (start 119.888 107.95) (end 118.11 107.95) (width 0.3048) (layer F.Cu) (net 5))
 (segment (start 120.396 108.458) (end 119.888 107.95) (width 0.3048) (layer F.Cu) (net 5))
 (segment (start 120.396 109.22) (end 120.396 108.458) (width 0.3048) (layer F.Cu) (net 5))
 (segment (start 121.031 109.855) (end 120.396 109.22) (width 0.3048) (layer F.Cu) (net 5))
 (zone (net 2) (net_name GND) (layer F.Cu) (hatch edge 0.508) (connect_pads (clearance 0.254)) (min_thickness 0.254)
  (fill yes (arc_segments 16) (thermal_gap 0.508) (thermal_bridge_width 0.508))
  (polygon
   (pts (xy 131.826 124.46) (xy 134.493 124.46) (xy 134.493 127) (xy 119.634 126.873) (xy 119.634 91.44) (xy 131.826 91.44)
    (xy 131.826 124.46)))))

